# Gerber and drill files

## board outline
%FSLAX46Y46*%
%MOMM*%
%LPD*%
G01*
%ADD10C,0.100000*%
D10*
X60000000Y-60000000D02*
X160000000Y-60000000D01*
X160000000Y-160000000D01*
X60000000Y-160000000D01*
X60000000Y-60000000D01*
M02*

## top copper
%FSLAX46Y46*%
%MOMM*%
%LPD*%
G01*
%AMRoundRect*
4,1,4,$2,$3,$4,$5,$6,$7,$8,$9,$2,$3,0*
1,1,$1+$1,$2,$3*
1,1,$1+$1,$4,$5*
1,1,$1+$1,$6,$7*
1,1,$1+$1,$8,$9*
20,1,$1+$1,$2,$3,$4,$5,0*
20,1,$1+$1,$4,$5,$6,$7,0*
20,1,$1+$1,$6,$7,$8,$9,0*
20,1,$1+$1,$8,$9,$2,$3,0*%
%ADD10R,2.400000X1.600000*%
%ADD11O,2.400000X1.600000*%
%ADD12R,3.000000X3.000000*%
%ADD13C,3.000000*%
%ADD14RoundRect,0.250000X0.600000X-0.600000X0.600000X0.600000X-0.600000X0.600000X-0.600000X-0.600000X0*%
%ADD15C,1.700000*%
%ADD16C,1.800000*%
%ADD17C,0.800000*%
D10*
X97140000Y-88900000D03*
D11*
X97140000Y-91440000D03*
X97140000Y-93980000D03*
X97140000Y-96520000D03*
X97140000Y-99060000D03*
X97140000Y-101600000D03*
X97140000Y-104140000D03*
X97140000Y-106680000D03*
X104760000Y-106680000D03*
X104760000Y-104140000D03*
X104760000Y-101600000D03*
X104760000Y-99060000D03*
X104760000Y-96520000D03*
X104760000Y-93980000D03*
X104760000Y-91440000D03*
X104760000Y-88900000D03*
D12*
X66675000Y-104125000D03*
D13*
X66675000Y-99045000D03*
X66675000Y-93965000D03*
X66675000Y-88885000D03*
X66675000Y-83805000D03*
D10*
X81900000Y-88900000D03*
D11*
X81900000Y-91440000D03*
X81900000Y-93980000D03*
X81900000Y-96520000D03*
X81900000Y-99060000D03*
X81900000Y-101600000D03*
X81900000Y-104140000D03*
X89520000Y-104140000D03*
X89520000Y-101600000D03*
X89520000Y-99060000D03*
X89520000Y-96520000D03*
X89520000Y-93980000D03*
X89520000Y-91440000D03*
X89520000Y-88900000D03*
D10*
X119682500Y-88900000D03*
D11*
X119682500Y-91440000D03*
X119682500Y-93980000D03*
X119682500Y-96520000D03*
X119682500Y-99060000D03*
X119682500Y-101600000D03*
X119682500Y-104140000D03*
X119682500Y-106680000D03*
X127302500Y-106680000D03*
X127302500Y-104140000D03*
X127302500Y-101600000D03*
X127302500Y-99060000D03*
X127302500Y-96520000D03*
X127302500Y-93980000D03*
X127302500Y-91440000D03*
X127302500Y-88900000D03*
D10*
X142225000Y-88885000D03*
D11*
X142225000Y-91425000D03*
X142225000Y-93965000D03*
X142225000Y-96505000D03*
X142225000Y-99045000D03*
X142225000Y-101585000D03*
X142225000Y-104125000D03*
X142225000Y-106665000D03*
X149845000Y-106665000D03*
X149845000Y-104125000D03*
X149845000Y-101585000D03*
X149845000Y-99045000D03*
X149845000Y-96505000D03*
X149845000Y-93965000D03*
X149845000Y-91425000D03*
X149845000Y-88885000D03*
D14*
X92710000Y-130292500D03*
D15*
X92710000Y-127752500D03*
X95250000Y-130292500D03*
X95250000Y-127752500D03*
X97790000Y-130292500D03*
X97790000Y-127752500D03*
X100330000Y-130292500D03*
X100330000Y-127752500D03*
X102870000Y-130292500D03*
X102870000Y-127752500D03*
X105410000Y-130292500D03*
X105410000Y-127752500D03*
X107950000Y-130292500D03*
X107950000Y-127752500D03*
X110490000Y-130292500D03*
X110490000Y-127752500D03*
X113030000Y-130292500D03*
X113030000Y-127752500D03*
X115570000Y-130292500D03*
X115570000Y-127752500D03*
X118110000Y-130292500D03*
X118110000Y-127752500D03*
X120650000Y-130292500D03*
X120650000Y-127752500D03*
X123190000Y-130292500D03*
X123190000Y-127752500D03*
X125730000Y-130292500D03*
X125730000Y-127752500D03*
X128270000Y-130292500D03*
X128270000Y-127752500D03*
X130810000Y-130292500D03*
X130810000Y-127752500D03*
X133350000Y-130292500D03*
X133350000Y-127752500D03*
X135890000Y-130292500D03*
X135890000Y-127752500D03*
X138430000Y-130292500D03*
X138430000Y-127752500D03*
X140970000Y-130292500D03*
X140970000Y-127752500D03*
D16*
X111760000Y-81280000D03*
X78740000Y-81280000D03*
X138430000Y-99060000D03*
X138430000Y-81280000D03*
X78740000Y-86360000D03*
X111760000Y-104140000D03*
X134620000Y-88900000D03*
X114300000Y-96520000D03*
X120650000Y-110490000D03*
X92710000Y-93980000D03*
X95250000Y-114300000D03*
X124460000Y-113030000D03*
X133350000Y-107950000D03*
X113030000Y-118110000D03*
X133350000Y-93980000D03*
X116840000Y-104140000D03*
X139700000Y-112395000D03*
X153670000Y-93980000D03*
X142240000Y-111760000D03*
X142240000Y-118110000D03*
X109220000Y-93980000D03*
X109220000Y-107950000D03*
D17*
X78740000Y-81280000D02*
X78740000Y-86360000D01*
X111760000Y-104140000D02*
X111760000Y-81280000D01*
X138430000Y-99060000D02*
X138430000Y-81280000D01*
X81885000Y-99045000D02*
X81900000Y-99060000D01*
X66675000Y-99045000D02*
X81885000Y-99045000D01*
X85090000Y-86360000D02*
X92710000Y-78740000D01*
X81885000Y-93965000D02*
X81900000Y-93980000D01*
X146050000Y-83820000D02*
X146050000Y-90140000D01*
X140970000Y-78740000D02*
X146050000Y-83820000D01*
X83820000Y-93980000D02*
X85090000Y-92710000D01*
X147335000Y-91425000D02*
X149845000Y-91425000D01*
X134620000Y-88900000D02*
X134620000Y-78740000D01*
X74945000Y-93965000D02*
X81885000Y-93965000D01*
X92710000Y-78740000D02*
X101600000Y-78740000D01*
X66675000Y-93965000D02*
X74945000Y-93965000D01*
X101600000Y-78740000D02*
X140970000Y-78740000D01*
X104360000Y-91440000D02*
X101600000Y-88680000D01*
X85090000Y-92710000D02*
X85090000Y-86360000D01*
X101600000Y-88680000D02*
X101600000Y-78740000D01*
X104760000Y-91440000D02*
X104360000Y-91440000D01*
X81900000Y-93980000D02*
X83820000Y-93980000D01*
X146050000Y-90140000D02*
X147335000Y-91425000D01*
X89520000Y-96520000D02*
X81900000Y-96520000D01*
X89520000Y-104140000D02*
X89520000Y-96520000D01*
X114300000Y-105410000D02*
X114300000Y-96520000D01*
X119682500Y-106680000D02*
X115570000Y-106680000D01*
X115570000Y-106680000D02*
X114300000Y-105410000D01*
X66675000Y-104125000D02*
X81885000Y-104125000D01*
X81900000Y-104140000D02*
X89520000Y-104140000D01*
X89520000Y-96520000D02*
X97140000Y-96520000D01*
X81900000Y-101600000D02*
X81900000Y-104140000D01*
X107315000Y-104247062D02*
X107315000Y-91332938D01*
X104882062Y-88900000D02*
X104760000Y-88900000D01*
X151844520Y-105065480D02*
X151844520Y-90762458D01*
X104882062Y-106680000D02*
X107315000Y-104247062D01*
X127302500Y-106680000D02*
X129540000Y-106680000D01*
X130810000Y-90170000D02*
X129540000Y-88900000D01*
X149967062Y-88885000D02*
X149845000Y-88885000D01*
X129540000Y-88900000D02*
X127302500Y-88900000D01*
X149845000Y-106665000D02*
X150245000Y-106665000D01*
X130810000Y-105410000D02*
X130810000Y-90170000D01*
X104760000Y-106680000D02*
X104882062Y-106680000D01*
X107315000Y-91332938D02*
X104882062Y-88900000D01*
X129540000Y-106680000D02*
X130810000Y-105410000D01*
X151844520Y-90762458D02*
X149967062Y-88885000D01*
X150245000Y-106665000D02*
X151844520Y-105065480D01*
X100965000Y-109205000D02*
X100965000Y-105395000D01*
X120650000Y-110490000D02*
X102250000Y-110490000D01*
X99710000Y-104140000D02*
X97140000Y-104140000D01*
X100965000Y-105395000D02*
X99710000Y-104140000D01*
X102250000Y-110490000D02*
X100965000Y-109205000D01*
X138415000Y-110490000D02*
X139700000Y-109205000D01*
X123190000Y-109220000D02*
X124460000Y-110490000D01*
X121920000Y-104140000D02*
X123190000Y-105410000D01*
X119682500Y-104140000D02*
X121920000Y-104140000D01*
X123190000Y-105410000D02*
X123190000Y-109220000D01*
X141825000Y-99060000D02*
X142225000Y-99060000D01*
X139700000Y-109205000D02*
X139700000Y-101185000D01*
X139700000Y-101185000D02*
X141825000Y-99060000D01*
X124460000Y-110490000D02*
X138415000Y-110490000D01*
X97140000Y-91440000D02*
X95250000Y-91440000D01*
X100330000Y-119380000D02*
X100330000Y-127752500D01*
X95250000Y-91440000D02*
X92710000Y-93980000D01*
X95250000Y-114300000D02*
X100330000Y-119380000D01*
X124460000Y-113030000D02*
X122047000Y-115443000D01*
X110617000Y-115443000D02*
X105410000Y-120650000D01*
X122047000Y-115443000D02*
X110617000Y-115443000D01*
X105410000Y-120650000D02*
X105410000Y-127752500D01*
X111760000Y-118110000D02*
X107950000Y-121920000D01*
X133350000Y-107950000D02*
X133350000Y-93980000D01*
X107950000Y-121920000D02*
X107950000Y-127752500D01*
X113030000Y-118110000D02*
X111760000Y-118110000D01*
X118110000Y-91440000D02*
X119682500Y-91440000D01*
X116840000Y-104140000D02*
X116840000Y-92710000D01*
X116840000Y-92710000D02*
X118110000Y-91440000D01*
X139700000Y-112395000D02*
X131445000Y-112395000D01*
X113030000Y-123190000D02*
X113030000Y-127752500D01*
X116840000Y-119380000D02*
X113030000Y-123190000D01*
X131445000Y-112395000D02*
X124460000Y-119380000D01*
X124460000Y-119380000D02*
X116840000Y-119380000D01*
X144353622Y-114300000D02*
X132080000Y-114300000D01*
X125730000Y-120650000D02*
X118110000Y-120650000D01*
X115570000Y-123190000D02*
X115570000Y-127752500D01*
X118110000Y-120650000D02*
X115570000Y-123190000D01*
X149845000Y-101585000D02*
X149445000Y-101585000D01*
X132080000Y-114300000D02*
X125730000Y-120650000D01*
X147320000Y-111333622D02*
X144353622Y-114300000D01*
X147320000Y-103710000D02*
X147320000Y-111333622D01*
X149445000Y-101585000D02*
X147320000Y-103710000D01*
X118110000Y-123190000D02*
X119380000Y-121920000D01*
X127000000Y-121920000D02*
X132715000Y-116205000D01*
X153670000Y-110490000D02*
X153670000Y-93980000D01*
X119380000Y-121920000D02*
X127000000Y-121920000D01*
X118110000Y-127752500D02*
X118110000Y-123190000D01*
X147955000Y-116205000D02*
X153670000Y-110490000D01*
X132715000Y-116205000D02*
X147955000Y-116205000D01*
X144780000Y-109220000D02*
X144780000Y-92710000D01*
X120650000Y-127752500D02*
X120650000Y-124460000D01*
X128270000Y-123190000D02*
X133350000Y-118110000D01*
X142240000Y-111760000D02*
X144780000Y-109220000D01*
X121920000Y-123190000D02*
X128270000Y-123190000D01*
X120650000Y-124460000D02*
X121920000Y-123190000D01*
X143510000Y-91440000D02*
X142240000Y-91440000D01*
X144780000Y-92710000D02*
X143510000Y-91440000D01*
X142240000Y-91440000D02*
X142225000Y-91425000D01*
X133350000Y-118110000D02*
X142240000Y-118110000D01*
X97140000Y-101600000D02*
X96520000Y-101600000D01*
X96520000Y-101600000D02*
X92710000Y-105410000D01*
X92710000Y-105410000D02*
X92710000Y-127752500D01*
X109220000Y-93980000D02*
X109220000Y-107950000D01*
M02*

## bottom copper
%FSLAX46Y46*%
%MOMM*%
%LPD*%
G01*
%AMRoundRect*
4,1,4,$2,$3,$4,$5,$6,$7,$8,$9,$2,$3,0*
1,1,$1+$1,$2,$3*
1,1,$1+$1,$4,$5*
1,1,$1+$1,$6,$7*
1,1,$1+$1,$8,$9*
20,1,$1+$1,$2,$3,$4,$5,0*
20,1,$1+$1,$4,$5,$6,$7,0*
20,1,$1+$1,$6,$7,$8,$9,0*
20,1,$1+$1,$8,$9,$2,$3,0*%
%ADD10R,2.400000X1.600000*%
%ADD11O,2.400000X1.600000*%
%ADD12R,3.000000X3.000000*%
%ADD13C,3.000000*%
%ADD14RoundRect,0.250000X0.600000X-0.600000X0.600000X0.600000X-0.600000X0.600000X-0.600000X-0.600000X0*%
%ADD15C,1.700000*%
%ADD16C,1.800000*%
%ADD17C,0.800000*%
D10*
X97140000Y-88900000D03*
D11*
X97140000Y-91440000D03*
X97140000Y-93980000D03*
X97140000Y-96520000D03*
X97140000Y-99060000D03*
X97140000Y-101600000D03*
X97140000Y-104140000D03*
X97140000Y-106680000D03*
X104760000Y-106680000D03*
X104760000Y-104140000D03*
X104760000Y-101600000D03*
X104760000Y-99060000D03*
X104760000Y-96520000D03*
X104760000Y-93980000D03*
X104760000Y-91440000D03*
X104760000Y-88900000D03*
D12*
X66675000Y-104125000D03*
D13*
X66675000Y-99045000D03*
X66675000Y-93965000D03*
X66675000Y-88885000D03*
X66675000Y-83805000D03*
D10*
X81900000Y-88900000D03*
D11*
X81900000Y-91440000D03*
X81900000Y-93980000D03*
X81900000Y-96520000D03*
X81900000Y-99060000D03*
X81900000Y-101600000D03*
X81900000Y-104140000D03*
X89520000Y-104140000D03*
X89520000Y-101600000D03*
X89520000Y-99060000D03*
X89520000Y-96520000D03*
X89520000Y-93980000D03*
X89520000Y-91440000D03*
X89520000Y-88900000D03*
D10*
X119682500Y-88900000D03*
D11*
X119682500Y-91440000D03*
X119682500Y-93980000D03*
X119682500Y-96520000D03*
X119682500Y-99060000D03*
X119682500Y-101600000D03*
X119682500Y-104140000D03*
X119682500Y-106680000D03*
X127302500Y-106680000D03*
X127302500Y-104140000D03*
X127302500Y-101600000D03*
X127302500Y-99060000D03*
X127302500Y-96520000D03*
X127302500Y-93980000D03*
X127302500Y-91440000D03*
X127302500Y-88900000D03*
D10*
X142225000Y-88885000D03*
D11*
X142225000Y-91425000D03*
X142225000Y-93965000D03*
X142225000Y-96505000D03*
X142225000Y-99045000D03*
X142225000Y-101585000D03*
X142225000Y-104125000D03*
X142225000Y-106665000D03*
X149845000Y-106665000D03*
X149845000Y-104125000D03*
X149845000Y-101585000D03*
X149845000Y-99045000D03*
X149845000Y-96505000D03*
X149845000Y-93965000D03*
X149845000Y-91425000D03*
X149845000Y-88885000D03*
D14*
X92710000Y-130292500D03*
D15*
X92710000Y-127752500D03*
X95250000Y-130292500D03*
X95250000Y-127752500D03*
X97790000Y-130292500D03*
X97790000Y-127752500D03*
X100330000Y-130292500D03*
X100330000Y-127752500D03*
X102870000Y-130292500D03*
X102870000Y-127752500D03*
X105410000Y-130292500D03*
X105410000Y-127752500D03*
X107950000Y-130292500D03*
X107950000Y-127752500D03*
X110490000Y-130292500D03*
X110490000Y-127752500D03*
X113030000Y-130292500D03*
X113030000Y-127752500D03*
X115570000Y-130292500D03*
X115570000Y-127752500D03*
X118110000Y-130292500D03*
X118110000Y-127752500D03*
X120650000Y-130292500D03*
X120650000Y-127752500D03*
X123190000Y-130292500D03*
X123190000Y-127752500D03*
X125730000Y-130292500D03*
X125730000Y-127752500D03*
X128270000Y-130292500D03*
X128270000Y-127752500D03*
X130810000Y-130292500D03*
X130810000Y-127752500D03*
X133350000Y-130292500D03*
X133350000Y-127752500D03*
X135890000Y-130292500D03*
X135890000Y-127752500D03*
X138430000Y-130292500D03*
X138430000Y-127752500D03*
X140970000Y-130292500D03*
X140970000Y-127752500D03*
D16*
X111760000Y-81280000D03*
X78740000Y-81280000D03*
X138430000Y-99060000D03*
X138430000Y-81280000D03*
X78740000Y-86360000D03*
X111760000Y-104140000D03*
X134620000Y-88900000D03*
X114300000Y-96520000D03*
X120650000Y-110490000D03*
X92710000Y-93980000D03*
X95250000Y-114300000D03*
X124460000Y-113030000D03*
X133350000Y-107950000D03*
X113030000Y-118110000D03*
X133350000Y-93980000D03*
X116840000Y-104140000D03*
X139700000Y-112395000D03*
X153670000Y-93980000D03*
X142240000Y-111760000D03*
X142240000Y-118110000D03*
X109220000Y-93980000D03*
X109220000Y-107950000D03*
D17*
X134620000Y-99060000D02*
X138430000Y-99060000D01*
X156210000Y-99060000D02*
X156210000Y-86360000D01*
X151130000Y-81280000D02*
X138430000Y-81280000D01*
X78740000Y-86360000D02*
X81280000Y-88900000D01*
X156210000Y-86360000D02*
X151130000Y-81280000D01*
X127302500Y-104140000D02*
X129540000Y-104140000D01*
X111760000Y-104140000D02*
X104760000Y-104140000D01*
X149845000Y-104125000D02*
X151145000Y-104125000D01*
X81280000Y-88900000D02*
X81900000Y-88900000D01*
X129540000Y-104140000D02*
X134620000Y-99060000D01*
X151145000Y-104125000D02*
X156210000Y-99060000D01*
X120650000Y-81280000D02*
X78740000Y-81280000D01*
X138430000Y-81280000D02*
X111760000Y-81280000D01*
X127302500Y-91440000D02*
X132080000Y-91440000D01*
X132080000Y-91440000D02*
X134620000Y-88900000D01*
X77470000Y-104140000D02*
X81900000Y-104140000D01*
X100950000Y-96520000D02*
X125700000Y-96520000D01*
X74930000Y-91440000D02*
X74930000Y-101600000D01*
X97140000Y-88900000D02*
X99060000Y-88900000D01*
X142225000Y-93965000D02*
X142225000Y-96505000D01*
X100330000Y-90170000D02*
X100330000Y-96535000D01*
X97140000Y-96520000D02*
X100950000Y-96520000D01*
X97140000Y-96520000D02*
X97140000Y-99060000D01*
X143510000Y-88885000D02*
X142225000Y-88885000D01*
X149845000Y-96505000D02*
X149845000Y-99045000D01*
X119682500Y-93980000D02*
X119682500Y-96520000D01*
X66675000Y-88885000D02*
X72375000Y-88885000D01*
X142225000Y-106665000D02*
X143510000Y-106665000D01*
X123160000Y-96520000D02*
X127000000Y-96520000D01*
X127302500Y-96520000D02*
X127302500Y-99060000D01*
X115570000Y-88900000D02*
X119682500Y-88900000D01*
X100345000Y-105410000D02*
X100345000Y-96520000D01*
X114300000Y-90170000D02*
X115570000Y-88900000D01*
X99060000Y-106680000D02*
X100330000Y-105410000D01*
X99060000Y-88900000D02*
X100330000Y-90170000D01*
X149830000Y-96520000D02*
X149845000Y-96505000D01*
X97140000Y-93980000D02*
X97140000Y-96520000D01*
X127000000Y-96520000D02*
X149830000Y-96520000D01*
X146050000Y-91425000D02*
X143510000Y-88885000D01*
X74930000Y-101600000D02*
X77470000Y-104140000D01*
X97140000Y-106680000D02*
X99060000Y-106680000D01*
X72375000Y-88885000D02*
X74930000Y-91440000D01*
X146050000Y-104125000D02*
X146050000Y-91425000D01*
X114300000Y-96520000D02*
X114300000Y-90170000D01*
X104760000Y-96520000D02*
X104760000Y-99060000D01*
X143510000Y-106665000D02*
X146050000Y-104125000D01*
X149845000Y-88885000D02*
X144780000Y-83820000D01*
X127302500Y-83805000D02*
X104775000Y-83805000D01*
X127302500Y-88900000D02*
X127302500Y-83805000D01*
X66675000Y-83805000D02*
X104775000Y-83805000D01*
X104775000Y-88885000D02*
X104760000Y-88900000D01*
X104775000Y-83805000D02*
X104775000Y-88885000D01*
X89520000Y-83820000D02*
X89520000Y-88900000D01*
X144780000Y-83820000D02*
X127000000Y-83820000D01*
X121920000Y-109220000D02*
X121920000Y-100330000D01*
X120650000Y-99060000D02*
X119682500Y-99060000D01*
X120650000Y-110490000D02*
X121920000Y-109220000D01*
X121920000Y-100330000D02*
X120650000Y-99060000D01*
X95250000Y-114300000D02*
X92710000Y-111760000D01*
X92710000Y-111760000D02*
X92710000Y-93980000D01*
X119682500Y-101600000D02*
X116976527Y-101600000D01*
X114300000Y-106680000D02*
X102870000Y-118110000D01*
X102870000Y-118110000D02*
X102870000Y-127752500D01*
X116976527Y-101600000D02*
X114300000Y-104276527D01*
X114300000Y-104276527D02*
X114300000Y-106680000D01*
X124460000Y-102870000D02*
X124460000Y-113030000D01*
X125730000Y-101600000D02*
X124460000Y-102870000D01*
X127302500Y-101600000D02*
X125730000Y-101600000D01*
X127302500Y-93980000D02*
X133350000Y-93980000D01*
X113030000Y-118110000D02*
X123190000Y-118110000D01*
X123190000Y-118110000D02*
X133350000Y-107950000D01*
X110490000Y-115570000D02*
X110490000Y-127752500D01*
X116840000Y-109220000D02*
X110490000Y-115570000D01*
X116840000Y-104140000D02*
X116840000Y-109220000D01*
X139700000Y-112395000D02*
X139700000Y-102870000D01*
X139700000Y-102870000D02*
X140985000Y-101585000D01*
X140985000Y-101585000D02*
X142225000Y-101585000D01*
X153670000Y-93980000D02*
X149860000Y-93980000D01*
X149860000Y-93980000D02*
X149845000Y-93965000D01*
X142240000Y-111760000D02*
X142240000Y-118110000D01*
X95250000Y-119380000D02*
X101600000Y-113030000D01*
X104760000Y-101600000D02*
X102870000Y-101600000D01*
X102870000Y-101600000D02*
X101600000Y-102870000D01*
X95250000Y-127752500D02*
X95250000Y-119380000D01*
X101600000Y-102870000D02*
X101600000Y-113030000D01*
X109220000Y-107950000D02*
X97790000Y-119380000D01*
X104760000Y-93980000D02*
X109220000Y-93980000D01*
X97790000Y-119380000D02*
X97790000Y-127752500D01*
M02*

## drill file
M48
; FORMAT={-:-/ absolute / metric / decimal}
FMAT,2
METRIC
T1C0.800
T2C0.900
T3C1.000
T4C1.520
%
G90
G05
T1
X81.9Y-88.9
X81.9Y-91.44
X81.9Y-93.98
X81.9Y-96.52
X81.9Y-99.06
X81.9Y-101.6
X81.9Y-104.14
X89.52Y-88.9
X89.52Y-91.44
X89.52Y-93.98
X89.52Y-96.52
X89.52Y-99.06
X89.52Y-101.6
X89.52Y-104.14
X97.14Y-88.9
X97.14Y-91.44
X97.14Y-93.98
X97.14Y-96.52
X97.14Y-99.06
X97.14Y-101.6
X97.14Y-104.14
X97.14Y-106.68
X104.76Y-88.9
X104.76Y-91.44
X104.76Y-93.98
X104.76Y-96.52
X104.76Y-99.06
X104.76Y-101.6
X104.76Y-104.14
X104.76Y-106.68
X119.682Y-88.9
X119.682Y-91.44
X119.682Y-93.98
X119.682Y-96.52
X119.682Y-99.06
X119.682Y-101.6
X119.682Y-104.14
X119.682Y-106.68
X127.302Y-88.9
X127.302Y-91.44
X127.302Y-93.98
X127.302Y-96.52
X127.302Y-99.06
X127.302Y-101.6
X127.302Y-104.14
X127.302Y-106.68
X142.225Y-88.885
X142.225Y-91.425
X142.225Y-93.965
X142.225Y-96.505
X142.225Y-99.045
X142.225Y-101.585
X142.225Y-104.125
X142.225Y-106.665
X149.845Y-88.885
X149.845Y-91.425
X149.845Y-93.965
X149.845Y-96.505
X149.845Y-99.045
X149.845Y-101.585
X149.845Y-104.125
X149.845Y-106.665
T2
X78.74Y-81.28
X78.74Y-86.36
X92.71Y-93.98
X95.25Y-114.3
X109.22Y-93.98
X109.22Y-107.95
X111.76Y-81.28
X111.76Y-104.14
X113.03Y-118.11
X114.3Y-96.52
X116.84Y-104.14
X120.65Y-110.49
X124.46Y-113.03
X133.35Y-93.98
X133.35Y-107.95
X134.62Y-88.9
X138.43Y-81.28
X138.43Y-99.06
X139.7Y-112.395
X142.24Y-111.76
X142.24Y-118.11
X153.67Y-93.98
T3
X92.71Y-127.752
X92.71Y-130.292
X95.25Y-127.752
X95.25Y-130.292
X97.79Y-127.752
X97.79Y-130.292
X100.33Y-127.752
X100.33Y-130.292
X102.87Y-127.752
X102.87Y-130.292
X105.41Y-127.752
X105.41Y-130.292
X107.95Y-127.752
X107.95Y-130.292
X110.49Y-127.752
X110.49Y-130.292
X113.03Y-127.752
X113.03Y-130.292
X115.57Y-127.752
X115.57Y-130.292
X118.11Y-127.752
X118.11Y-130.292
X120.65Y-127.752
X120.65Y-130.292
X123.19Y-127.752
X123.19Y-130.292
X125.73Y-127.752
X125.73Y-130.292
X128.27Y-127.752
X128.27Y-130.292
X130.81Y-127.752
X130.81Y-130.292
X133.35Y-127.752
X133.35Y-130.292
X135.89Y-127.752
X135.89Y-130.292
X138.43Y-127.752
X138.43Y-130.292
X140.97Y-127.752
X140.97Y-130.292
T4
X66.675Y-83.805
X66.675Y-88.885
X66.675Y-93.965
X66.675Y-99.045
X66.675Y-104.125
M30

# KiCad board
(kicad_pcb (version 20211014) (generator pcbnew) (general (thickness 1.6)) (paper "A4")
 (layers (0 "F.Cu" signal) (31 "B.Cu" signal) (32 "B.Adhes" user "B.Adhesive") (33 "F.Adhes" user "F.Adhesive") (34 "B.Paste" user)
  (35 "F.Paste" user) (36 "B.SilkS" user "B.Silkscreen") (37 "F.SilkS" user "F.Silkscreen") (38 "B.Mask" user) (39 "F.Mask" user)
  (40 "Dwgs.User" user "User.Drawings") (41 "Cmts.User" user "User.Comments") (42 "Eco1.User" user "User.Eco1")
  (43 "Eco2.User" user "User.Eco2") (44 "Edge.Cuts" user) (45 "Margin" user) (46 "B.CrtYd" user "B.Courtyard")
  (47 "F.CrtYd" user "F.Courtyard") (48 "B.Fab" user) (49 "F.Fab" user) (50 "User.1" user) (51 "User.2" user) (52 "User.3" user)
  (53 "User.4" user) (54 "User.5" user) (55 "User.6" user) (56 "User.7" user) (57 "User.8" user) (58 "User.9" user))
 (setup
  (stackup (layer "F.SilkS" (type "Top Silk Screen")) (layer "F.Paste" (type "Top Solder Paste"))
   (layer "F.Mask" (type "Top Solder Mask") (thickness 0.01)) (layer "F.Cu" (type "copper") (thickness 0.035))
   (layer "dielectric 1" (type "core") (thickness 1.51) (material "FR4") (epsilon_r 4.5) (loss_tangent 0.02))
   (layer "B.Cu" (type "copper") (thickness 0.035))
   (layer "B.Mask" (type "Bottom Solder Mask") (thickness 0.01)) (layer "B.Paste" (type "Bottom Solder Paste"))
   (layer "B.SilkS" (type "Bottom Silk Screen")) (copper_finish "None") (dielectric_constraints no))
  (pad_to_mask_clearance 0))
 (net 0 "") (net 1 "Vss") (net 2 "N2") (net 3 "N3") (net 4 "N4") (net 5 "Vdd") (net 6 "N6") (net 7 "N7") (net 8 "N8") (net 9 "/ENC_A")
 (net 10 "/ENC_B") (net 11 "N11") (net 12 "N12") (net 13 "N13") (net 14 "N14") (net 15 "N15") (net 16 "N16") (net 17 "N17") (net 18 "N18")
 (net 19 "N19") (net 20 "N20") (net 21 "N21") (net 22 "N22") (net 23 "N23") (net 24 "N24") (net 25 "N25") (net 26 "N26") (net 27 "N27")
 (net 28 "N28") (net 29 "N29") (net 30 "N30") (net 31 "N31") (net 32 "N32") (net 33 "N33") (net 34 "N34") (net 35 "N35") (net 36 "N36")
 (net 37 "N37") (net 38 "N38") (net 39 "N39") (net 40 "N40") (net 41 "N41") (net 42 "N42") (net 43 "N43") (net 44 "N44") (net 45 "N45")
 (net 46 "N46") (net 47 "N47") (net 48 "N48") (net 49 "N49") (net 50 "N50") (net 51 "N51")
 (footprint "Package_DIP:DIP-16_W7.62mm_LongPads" (layer "F.Cu") (at 97.14 88.9)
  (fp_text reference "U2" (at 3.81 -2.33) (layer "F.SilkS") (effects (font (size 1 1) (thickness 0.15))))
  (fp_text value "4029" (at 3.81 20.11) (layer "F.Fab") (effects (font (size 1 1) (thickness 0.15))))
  (pad "1" thru_hole rect (at 0 0) (size 2.4 1.6) (drill 0.8) (layers *.Cu *.Mask) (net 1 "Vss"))
  (pad "2" thru_hole oval (at 0 2.54) (size 2.4 1.6) (drill 0.8) (layers *.Cu *.Mask) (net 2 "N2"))
  (pad "3" thru_hole oval (at 0 5.08) (size 2.4 1.6) (drill 0.8) (layers *.Cu *.Mask) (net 1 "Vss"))
  (pad "4" thru_hole oval (at 0 7.62) (size 2.4 1.6) (drill 0.8) (layers *.Cu *.Mask) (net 1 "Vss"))
  (pad "5" thru_hole oval (at 0 10.16) (size 2.4 1.6) (drill 0.8) (layers *.Cu *.Mask) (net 1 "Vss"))
  (pad "6" thru_hole oval (at 0 12.7) (size 2.4 1.6) (drill 0.8) (layers *.Cu *.Mask) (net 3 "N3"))
  (pad "7" thru_hole oval (at 0 15.24) (size 2.4 1.6) (drill 0.8) (layers *.Cu *.Mask) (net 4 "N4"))
  (pad "8" thru_hole oval (at 0 17.78) (size 2.4 1.6) (drill 0.8) (layers *.Cu *.Mask) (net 1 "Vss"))
  (pad "9" thru_hole oval (at 7.62 17.78) (size 2.4 1.6) (drill 0.8) (layers *.Cu *.Mask) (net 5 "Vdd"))
  (pad "10" thru_hole oval (at 7.62 15.24) (size 2.4 1.6) (drill 0.8) (layers *.Cu *.Mask) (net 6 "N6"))
  (pad "11" thru_hole oval (at 7.62 12.7) (size 2.4 1.6) (drill 0.8) (layers *.Cu *.Mask) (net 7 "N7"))
  (pad "12" thru_hole oval (at 7.62 10.16) (size 2.4 1.6) (drill 0.8) (layers *.Cu *.Mask) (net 1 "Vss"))
  (pad "13" thru_hole oval (at 7.62 7.62) (size 2.4 1.6) (drill 0.8) (layers *.Cu *.Mask) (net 1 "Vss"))
  (pad "14" thru_hole oval (at 7.62 5.08) (size 2.4 1.6) (drill 0.8) (layers *.Cu *.Mask) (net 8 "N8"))
  (pad "15" thru_hole oval (at 7.62 2.54) (size 2.4 1.6) (drill 0.8) (layers *.Cu *.Mask) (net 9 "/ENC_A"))
  (pad "16" thru_hole oval (at 7.62 0) (size 2.4 1.6) (drill 0.8) (layers *.Cu *.Mask) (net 5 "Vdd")))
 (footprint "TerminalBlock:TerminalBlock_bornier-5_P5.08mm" (layer "F.Cu") (at 66.675 104.125 90)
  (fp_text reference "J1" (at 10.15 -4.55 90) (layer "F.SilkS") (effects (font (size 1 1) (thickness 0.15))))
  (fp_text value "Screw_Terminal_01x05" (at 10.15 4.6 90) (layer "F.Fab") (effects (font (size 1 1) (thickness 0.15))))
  (pad "1" thru_hole rect (at 0 0 90) (size 3 3) (drill 1.52) (layers *.Cu *.Mask) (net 1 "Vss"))
  (pad "2" thru_hole circle (at 5.08 0 90) (size 3 3) (drill 1.52) (layers *.Cu *.Mask) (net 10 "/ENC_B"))
  (pad "3" thru_hole circle (at 10.16 0 90) (size 3 3) (drill 1.52) (layers *.Cu *.Mask) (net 9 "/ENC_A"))
  (pad "4" thru_hole circle (at 15.24 0 90) (size 3 3) (drill 1.52) (layers *.Cu *.Mask) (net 1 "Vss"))
  (pad "5" thru_hole circle (at 20.32 0 90) (size 3 3) (drill 1.52) (layers *.Cu *.Mask) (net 5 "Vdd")))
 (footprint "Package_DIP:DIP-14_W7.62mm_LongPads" (layer "F.Cu") (at 81.9 88.9)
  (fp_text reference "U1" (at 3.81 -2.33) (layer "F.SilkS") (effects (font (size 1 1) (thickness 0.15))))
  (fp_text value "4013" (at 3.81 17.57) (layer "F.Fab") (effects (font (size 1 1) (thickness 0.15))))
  (pad "1" thru_hole rect (at 0 0) (size 2.4 1.6) (drill 0.8) (layers *.Cu *.Mask) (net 6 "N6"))
  (pad "2" thru_hole oval (at 0 2.54) (size 2.4 1.6) (drill 0.8) (layers *.Cu *.Mask) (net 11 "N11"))
  (pad "3" thru_hole oval (at 0 5.08) (size 2.4 1.6) (drill 0.8) (layers *.Cu *.Mask) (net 9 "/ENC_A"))
  (pad "4" thru_hole oval (at 0 7.62) (size 2.4 1.6) (drill 0.8) (layers *.Cu *.Mask) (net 1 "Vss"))
  (pad "5" thru_hole oval (at 0 10.16) (size 2.4 1.6) (drill 0.8) (layers *.Cu *.Mask) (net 10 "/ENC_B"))
  (pad "6" thru_hole oval (at 0 12.7) (size 2.4 1.6) (drill 0.8) (layers *.Cu *.Mask) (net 1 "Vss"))
  (pad "7" thru_hole oval (at 0 15.24) (size 2.4 1.6) (drill 0.8) (layers *.Cu *.Mask) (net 1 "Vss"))
  (pad "8" thru_hole oval (at 7.62 15.24) (size 2.4 1.6) (drill 0.8) (layers *.Cu *.Mask) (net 1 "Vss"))
  (pad "9" thru_hole oval (at 7.62 12.7) (size 2.4 1.6) (drill 0.8) (layers *.Cu *.Mask) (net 1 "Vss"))
  (pad "10" thru_hole oval (at 7.62 10.16) (size 2.4 1.6) (drill 0.8) (layers *.Cu *.Mask) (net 1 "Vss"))
  (pad "11" thru_hole oval (at 7.62 7.62) (size 2.4 1.6) (drill 0.8) (layers *.Cu *.Mask) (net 1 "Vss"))
  (pad "12" thru_hole oval (at 7.62 5.08) (size 2.4 1.6) (drill 0.8) (layers *.Cu *.Mask) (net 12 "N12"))
  (pad "13" thru_hole oval (at 7.62 2.54) (size 2.4 1.6) (drill 0.8) (layers *.Cu *.Mask) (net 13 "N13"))
  (pad "14" thru_hole oval (at 7.62 0) (size 2.4 1.6) (drill 0.8) (layers *.Cu *.Mask) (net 5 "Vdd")))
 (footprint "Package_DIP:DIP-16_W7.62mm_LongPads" (layer "F.Cu") (at 119.6825 88.9)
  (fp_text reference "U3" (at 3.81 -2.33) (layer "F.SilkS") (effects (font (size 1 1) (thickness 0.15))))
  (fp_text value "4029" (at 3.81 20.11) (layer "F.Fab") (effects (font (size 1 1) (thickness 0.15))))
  (pad "1" thru_hole rect (at 0 0) (size 2.4 1.6) (drill 0.8) (layers *.Cu *.Mask) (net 1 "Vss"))
  (pad "2" thru_hole oval (at 0 2.54) (size 2.4 1.6) (drill 0.8) (layers *.Cu *.Mask) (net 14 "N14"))
  (pad "3" thru_hole oval (at 0 5.08) (size 2.4 1.6) (drill 0.8) (layers *.Cu *.Mask) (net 1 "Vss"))
  (pad "4" thru_hole oval (at 0 7.62) (size 2.4 1.6) (drill 0.8) (layers *.Cu *.Mask) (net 1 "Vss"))
  (pad "5" thru_hole oval (at 0 10.16) (size 2.4 1.6) (drill 0.8) (layers *.Cu *.Mask) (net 4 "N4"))
  (pad "6" thru_hole oval (at 0 12.7) (size 2.4 1.6) (drill 0.8) (layers *.Cu *.Mask) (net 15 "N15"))
  (pad "7" thru_hole oval (at 0 15.24) (size 2.4 1.6) (drill 0.8) (layers *.Cu *.Mask) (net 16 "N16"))
  (pad "8" thru_hole oval (at 0 17.78) (size 2.4 1.6) (drill 0.8) (layers *.Cu *.Mask) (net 1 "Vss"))
  (pad "9" thru_hole oval (at 7.62 17.78) (size 2.4 1.6) (drill 0.8) (layers *.Cu *.Mask) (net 5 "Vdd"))
  (pad "10" thru_hole oval (at 7.62 15.24) (size 2.4 1.6) (drill 0.8) (layers *.Cu *.Mask) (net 6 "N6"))
  (pad "11" thru_hole oval (at 7.62 12.7) (size 2.4 1.6) (drill 0.8) (layers *.Cu *.Mask) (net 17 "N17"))
  (pad "12" thru_hole oval (at 7.62 10.16) (size 2.4 1.6) (drill 0.8) (layers *.Cu *.Mask) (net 1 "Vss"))
  (pad "13" thru_hole oval (at 7.62 7.62) (size 2.4 1.6) (drill 0.8) (layers *.Cu *.Mask) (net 1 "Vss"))
  (pad "14" thru_hole oval (at 7.62 5.08) (size 2.4 1.6) (drill 0.8) (layers *.Cu *.Mask) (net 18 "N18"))
  (pad "15" thru_hole oval (at 7.62 2.54) (size 2.4 1.6) (drill 0.8) (layers *.Cu *.Mask) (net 9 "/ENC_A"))
  (pad "16" thru_hole oval (at 7.62 0) (size 2.4 1.6) (drill 0.8) (layers *.Cu *.Mask) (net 5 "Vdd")))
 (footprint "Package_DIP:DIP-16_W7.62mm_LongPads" (layer "F.Cu") (at 142.225 88.885)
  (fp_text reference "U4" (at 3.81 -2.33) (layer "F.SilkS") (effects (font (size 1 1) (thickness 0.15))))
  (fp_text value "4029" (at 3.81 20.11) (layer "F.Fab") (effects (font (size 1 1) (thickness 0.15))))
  (pad "1" thru_hole rect (at 0 0) (size 2.4 1.6) (drill 0.8) (layers *.Cu *.Mask) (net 1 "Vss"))
  (pad "2" thru_hole oval (at 0 2.54) (size 2.4 1.6) (drill 0.8) (layers *.Cu *.Mask) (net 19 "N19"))
  (pad "3" thru_hole oval (at 0 5.08) (size 2.4 1.6) (drill 0.8) (layers *.Cu *.Mask) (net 1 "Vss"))
  (pad "4" thru_hole oval (at 0 7.62) (size 2.4 1.6) (drill 0.8) (layers *.Cu *.Mask) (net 1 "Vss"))
  (pad "5" thru_hole oval (at 0 10.16) (size 2.4 1.6) (drill 0.8) (layers *.Cu *.Mask) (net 16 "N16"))
  (pad "6" thru_hole oval (at 0 12.7) (size 2.4 1.6) (drill 0.8) (layers *.Cu *.Mask) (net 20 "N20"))
  (pad "7" thru_hole oval (at 0 15.24) (size 2.4 1.6) (drill 0.8) (layers *.Cu *.Mask) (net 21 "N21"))
  (pad "8" thru_hole oval (at 0 17.78) (size 2.4 1.6) (drill 0.8) (layers *.Cu *.Mask) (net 1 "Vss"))
  (pad "9" thru_hole oval (at 7.62 17.78) (size 2.4 1.6) (drill 0.8) (layers *.Cu *.Mask) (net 5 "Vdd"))
  (pad "10" thru_hole oval (at 7.62 15.24) (size 2.4 1.6) (drill 0.8) (layers *.Cu *.Mask) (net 6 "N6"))
  (pad "11" thru_hole oval (at 7.62 12.7) (size 2.4 1.6) (drill 0.8) (layers *.Cu *.Mask) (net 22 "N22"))
  (pad "12" thru_hole oval (at 7.62 10.16) (size 2.4 1.6) (drill 0.8) (layers *.Cu *.Mask) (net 1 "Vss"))
  (pad "13" thru_hole oval (at 7.62 7.62) (size 2.4 1.6) (drill 0.8) (layers *.Cu *.Mask) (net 1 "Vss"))
  (pad "14" thru_hole oval (at 7.62 5.08) (size 2.4 1.6) (drill 0.8) (layers *.Cu *.Mask) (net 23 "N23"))
  (pad "15" thru_hole oval (at 7.62 2.54) (size 2.4 1.6) (drill 0.8) (layers *.Cu *.Mask) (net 9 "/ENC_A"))
  (pad "16" thru_hole oval (at 7.62 0) (size 2.4 1.6) (drill 0.8) (layers *.Cu *.Mask) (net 5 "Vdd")))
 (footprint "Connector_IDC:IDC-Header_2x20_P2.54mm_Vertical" (layer "F.Cu") (at 92.71 130.2925 90)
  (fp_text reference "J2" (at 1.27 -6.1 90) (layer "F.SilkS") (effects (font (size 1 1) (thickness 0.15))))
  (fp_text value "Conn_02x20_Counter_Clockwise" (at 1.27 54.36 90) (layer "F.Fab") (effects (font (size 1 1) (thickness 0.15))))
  (pad "1" thru_hole roundrect (at 0 0 90) (size 1.7 1.7) (drill 1) (layers *.Cu *.Mask) (roundrect_rratio 0.147059) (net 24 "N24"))
  (pad "2" thru_hole circle (at 2.54 0 90) (size 1.7 1.7) (drill 1) (layers *.Cu *.Mask) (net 3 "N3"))
  (pad "3" thru_hole circle (at 0 2.54 90) (size 1.7 1.7) (drill 1) (layers *.Cu *.Mask) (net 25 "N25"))
  (pad "4" thru_hole circle (at 2.54 2.54 90) (size 1.7 1.7) (drill 1) (layers *.Cu *.Mask) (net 7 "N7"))
  (pad "5" thru_hole circle (at 0 5.08 90) (size 1.7 1.7) (drill 1) (layers *.Cu *.Mask) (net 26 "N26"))
  (pad "6" thru_hole circle (at 2.54 5.08 90) (size 1.7 1.7) (drill 1) (layers *.Cu *.Mask) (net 8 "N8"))
  (pad "7" thru_hole circle (at 0 7.62 90) (size 1.7 1.7) (drill 1) (layers *.Cu *.Mask) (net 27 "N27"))
  (pad "8" thru_hole circle (at 2.54 7.62 90) (size 1.7 1.7) (drill 1) (layers *.Cu *.Mask) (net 2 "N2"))
  (pad "9" thru_hole circle (at 0 10.16 90) (size 1.7 1.7) (drill 1) (layers *.Cu *.Mask) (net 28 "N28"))
  (pad "10" thru_hole circle (at 2.54 10.16 90) (size 1.7 1.7) (drill 1) (layers *.Cu *.Mask) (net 15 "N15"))
  (pad "11" thru_hole circle (at 0 12.7 90) (size 1.7 1.7) (drill 1) (layers *.Cu *.Mask) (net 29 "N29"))
  (pad "12" thru_hole circle (at 2.54 12.7 90) (size 1.7 1.7) (drill 1) (layers *.Cu *.Mask) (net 17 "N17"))
  (pad "13" thru_hole circle (at 0 15.24 90) (size 1.7 1.7) (drill 1) (layers *.Cu *.Mask) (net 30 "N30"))
  (pad "14" thru_hole circle (at 2.54 15.24 90) (size 1.7 1.7) (drill 1) (layers *.Cu *.Mask) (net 18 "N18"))
  (pad "15" thru_hole circle (at 0 17.78 90) (size 1.7 1.7) (drill 1) (layers *.Cu *.Mask) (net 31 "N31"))
  (pad "16" thru_hole circle (at 2.54 17.78 90) (size 1.7 1.7) (drill 1) (layers *.Cu *.Mask) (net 14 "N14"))
  (pad "17" thru_hole circle (at 0 20.32 90) (size 1.7 1.7) (drill 1) (layers *.Cu *.Mask) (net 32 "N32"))
  (pad "18" thru_hole circle (at 2.54 20.32 90) (size 1.7 1.7) (drill 1) (layers *.Cu *.Mask) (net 20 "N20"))
  (pad "19" thru_hole circle (at 0 22.86 90) (size 1.7 1.7) (drill 1) (layers *.Cu *.Mask) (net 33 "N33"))
  (pad "20" thru_hole circle (at 2.54 22.86 90) (size 1.7 1.7) (drill 1) (layers *.Cu *.Mask) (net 22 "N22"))
  (pad "21" thru_hole circle (at 0 25.4 90) (size 1.7 1.7) (drill 1) (layers *.Cu *.Mask) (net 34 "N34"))
  (pad "22" thru_hole circle (at 2.54 25.4 90) (size 1.7 1.7) (drill 1) (layers *.Cu *.Mask) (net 23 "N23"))
  (pad "23" thru_hole circle (at 0 27.94 90) (size 1.7 1.7) (drill 1) (layers *.Cu *.Mask) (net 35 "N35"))
  (pad "24" thru_hole circle (at 2.54 27.94 90) (size 1.7 1.7) (drill 1) (layers *.Cu *.Mask) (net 19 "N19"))
  (pad "25" thru_hole circle (at 0 30.48 90) (size 1.7 1.7) (drill 1) (layers *.Cu *.Mask) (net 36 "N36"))
  (pad "26" thru_hole circle (at 2.54 30.48 90) (size 1.7 1.7) (drill 1) (layers *.Cu *.Mask) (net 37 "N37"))
  (pad "27" thru_hole circle (at 0 33.02 90) (size 1.7 1.7) (drill 1) (layers *.Cu *.Mask) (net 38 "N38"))
  (pad "28" thru_hole circle (at 2.54 33.02 90) (size 1.7 1.7) (drill 1) (layers *.Cu *.Mask) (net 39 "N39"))
  (pad "29" thru_hole circle (at 0 35.56 90) (size 1.7 1.7) (drill 1) (layers *.Cu *.Mask) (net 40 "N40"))
  (pad "30" thru_hole circle (at 2.54 35.56 90) (size 1.7 1.7) (drill 1) (layers *.Cu *.Mask) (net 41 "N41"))
  (pad "31" thru_hole circle (at 0 38.1 90) (size 1.7 1.7) (drill 1) (layers *.Cu *.Mask) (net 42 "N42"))
  (pad "32" thru_hole circle (at 2.54 38.1 90) (size 1.7 1.7) (drill 1) (layers *.Cu *.Mask) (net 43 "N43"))
  (pad "33" thru_hole circle (at 0 40.64 90) (size 1.7 1.7) (drill 1) (layers *.Cu *.Mask) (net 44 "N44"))
  (pad "34" thru_hole circle (at 2.54 40.64 90) (size 1.7 1.7) (drill 1) (layers *.Cu *.Mask) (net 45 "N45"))
  (pad "35" thru_hole circle (at 0 43.18 90) (size 1.7 1.7) (drill 1) (layers *.Cu *.Mask) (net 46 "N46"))
  (pad "36" thru_hole circle (at 2.54 43.18 90) (size 1.7 1.7) (drill 1) (layers *.Cu *.Mask) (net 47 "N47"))
  (pad "37" thru_hole circle (at 0 45.72 90) (size 1.7 1.7) (drill 1) (layers *.Cu *.Mask) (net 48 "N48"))
  (pad "38" thru_hole circle (at 2.54 45.72 90) (size 1.7 1.7) (drill 1) (layers *.Cu *.Mask) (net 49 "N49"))
  (pad "39" thru_hole circle (at 0 48.26 90) (size 1.7 1.7) (drill 1) (layers *.Cu *.Mask) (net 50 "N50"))
  (pad "40" thru_hole circle (at 2.54 48.26 90) (size 1.7 1.7) (drill 1) (layers *.Cu *.Mask) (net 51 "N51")))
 (gr_rect (start 60 60) (end 160 160) (layer "Edge.Cuts") (width 0.1) (fill none))
 (segment (start 78.74 81.28) (end 78.74 86.36) (width 0.8) (layer "F.Cu") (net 6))
 (segment (start 111.76 104.14) (end 111.76 81.28) (width 0.8) (layer "F.Cu") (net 6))
 (segment (start 138.43 99.06) (end 138.43 81.28) (width 0.8) (layer "F.Cu") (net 6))
 (via (at 111.76 81.28) (size 1.8) (drill 0.9) (layers "F.Cu" "B.Cu") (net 6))
 (via (at 78.74 81.28) (size 1.8) (drill 0.9) (layers "F.Cu" "B.Cu") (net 6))
 (via (at 138.43 99.06) (size 1.8) (drill 0.9) (layers "F.Cu" "B.Cu") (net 6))
 (via (at 138.43 81.28) (size 1.8) (drill 0.9) (layers "F.Cu" "B.Cu") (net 6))
 (via (at 78.74 86.36) (size 1.8) (drill 0.9) (layers "F.Cu" "B.Cu") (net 6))
 (via (at 111.76 104.14) (size 1.8) (drill 0.9) (layers "F.Cu" "B.Cu") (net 6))
 (segment (start 134.62 99.06) (end 138.43 99.06) (width 0.8) (layer "B.Cu") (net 6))
 (segment (start 156.21 99.06) (end 156.21 86.36) (width 0.8) (layer "B.Cu") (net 6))
 (segment (start 151.13 81.28) (end 138.43 81.28) (width 0.8) (layer "B.Cu") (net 6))
 (segment (start 78.74 86.36) (end 81.28 88.9) (width 0.8) (layer "B.Cu") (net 6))
 (segment (start 156.21 86.36) (end 151.13 81.28) (width 0.8) (layer "B.Cu") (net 6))
 (segment (start 127.3025 104.14) (end 129.54 104.14) (width 0.8) (layer "B.Cu") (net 6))
 (segment (start 111.76 104.14) (end 104.76 104.14) (width 0.8) (layer "B.Cu") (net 6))
 (segment (start 149.845 104.125) (end 151.145 104.125) (width 0.8) (layer "B.Cu") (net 6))
 (segment (start 81.28 88.9) (end 81.9 88.9) (width 0.8) (layer "B.Cu") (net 6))
 (segment (start 129.54 104.14) (end 134.62 99.06) (width 0.8) (layer "B.Cu") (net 6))
 (segment (start 151.145 104.125) (end 156.21 99.06) (width 0.8) (layer "B.Cu") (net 6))
 (segment (start 120.65 81.28) (end 78.74 81.28) (width 0.8) (layer "B.Cu") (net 6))
 (segment (start 138.43 81.28) (end 111.76 81.28) (width 0.8) (layer "B.Cu") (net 6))
 (segment (start 81.885 99.045) (end 81.9 99.06) (width 0.8) (layer "F.Cu") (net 10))
 (segment (start 66.675 99.045) (end 81.885 99.045) (width 0.8) (layer "F.Cu") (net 10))
 (segment (start 85.09 86.36) (end 92.71 78.74) (width 0.8) (layer "F.Cu") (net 9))
 (segment (start 81.885 93.965) (end 81.9 93.98) (width 0.8) (layer "F.Cu") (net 9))
 (segment (start 146.05 83.82) (end 146.05 90.14) (width 0.8) (layer "F.Cu") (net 9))
 (segment (start 140.97 78.74) (end 146.05 83.82) (width 0.8) (layer "F.Cu") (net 9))
 (segment (start 83.82 93.98) (end 85.09 92.71) (width 0.8) (layer "F.Cu") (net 9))
 (segment (start 147.335 91.425) (end 149.845 91.425) (width 0.8) (layer "F.Cu") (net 9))
 (segment (start 134.62 88.9) (end 134.62 78.74) (width 0.8) (layer "F.Cu") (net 9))
 (segment (start 74.945 93.965) (end 81.885 93.965) (width 0.8) (layer "F.Cu") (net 9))
 (segment (start 92.71 78.74) (end 101.6 78.74) (width 0.8) (layer "F.Cu") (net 9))
 (segment (start 66.675 93.965) (end 74.945 93.965) (width 0.8) (layer "F.Cu") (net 9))
 (segment (start 101.6 78.74) (end 140.97 78.74) (width 0.8) (layer "F.Cu") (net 9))
 (segment (start 104.36 91.44) (end 101.6 88.68) (width 0.8) (layer "F.Cu") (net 9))
 (segment (start 85.09 92.71) (end 85.09 86.36) (width 0.8) (layer "F.Cu") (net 9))
 (segment (start 101.6 88.68) (end 101.6 78.74) (width 0.8) (layer "F.Cu") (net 9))
 (segment (start 104.76 91.44) (end 104.36 91.44) (width 0.8) (layer "F.Cu") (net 9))
 (segment (start 81.9 93.98) (end 83.82 93.98) (width 0.8) (layer "F.Cu") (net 9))
 (segment (start 146.05 90.14) (end 147.335 91.425) (width 0.8) (layer "F.Cu") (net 9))
 (via (at 134.62 88.9) (size 1.8) (drill 0.9) (layers "F.Cu" "B.Cu") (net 9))
 (segment (start 127.3025 91.44) (end 132.08 91.44) (width 0.8) (layer "B.Cu") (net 9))
 (segment (start 132.08 91.44) (end 134.62 88.9) (width 0.8) (layer "B.Cu") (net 9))
 (segment (start 89.52 96.52) (end 81.9 96.52) (width 0.8) (layer "F.Cu") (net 1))
 (segment (start 89.52 104.14) (end 89.52 96.52) (width 0.8) (layer "F.Cu") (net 1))
 (segment (start 114.3 105.41) (end 114.3 96.52) (width 0.8) (layer "F.Cu") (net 1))
 (segment (start 119.6825 106.68) (end 115.57 106.68) (width 0.8) (layer "F.Cu") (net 1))
 (segment (start 115.57 106.68) (end 114.3 105.41) (width 0.8) (layer "F.Cu") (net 1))
 (segment (start 66.675 104.125) (end 81.885 104.125) (width 0.8) (layer "F.Cu") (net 1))
 (segment (start 81.9 104.14) (end 89.52 104.14) (width 0.8) (layer "F.Cu") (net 1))
 (segment (start 89.52 96.52) (end 97.14 96.52) (width 0.8) (layer "F.Cu") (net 1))
 (segment (start 81.9 101.6) (end 81.9 104.14) (width 0.8) (layer "F.Cu") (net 1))
 (via (at 114.3 96.52) (size 1.8) (drill 0.9) (layers "F.Cu" "B.Cu") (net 1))
 (segment (start 77.47 104.14) (end 81.9 104.14) (width 0.8) (layer "B.Cu") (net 1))
 (segment (start 100.95 96.52) (end 125.7 96.52) (width 0.8) (layer "B.Cu") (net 1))
 (segment (start 74.93 91.44) (end 74.93 101.6) (width 0.8) (layer "B.Cu") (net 1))
 (segment (start 97.14 88.9) (end 99.06 88.9) (width 0.8) (layer "B.Cu") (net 1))
 (segment (start 142.225 93.965) (end 142.225 96.505) (width 0.8) (layer "B.Cu") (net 1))
 (segment (start 100.33 90.17) (end 100.33 96.535) (width 0.8) (layer "B.Cu") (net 1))
 (segment (start 97.14 96.52) (end 100.95 96.52) (width 0.8) (layer "B.Cu") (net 1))
 (segment (start 97.14 96.52) (end 97.14 99.06) (width 0.8) (layer "B.Cu") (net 1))
 (segment (start 143.51 88.885) (end 142.225 88.885) (width 0.8) (layer "B.Cu") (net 1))
 (segment (start 149.845 96.505) (end 149.845 99.045) (width 0.8) (layer "B.Cu") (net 1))
 (segment (start 119.6825 93.98) (end 119.6825 96.52) (width 0.8) (layer "B.Cu") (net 1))
 (segment (start 66.675 88.885) (end 72.375 88.885) (width 0.8) (layer "B.Cu") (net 1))
 (segment (start 142.225 106.665) (end 143.51 106.665) (width 0.8) (layer "B.Cu") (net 1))
 (segment (start 123.16 96.52) (end 127 96.52) (width 0.8) (layer "B.Cu") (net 1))
 (segment (start 127.3025 96.52) (end 127.3025 99.06) (width 0.8) (layer "B.Cu") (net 1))
 (segment (start 115.57 88.9) (end 119.6825 88.9) (width 0.8) (layer "B.Cu") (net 1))
 (segment (start 100.345 105.41) (end 100.345 96.52) (width 0.8) (layer "B.Cu") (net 1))
 (segment (start 114.3 90.17) (end 115.57 88.9) (width 0.8) (layer "B.Cu") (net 1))
 (segment (start 99.06 106.68) (end 100.33 105.41) (width 0.8) (layer "B.Cu") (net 1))
 (segment (start 99.06 88.9) (end 100.33 90.17) (width 0.8) (layer "B.Cu") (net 1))
 (segment (start 149.83 96.52) (end 149.845 96.505) (width 0.8) (layer "B.Cu") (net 1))
 (segment (start 97.14 93.98) (end 97.14 96.52) (width 0.8) (layer "B.Cu") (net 1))
 (segment (start 127 96.52) (end 149.83 96.52) (width 0.8) (layer "B.Cu") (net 1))
 (segment (start 146.05 91.425) (end 143.51 88.885) (width 0.8) (layer "B.Cu") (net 1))
 (segment (start 74.93 101.6) (end 77.47 104.14) (width 0.8) (layer "B.Cu") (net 1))
 (segment (start 97.14 106.68) (end 99.06 106.68) (width 0.8) (layer "B.Cu") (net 1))
 (segment (start 72.375 88.885) (end 74.93 91.44) (width 0.8) (layer "B.Cu") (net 1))
 (segment (start 146.05 104.125) (end 146.05 91.425) (width 0.8) (layer "B.Cu") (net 1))
 (segment (start 114.3 96.52) (end 114.3 90.17) (width 0.8) (layer "B.Cu") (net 1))
 (segment (start 104.76 96.52) (end 104.76 99.06) (width 0.8) (layer "B.Cu") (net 1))
 (segment (start 143.51 106.665) (end 146.05 104.125) (width 0.8) (layer "B.Cu") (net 1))
 (segment (start 107.315 104.247062) (end 107.315 91.332938) (width 0.8) (layer "F.Cu") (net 5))
 (segment (start 104.882062 88.9) (end 104.76 88.9) (width 0.8) (layer "F.Cu") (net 5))
 (segment (start 151.84452 105.06548) (end 151.84452 90.762458) (width 0.8) (layer "F.Cu") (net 5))
 (segment (start 104.882062 106.68) (end 107.315 104.247062) (width 0.8) (layer "F.Cu") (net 5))
 (segment (start 127.3025 106.68) (end 129.54 106.68) (width 0.8) (layer "F.Cu") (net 5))
 (segment (start 130.81 90.17) (end 129.54 88.9) (width 0.8) (layer "F.Cu") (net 5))
 (segment (start 149.967062 88.885) (end 149.845 88.885) (width 0.8) (layer "F.Cu") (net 5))
 (segment (start 129.54 88.9) (end 127.3025 88.9) (width 0.8) (layer "F.Cu") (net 5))
 (segment (start 149.845 106.665) (end 150.245 106.665) (width 0.8) (layer "F.Cu") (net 5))
 (segment (start 130.81 105.41) (end 130.81 90.17) (width 0.8) (layer "F.Cu") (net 5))
 (segment (start 104.76 106.68) (end 104.882062 106.68) (width 0.8) (layer "F.Cu") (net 5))
 (segment (start 107.315 91.332938) (end 104.882062 88.9) (width 0.8) (layer "F.Cu") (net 5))
 (segment (start 129.54 106.68) (end 130.81 105.41) (width 0.8) (layer "F.Cu") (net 5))
 (segment (start 151.84452 90.762458) (end 149.967062 88.885) (width 0.8) (layer "F.Cu") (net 5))
 (segment (start 150.245 106.665) (end 151.84452 105.06548) (width 0.8) (layer "F.Cu") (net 5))
 (segment (start 149.845 88.885) (end 144.78 83.82) (width 0.8) (layer "B.Cu") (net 5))
 (segment (start 127.3025 83.805) (end 104.775 83.805) (width 0.8) (layer "B.Cu") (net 5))
 (segment (start 127.3025 88.9) (end 127.3025 83.805) (width 0.8) (layer "B.Cu") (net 5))
 (segment (start 66.675 83.805) (end 104.775 83.805) (width 0.8) (layer "B.Cu") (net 5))
 (segment (start 104.775 88.885) (end 104.76 88.9) (width 0.8) (layer "B.Cu") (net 5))
 (segment (start 104.775 83.805) (end 104.775 88.885) (width 0.8) (layer "B.Cu") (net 5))
 (segment (start 89.52 83.82) (end 89.52 88.9) (width 0.8) (layer "B.Cu") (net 5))
 (segment (start 144.78 83.82) (end 127 83.82) (width 0.8) (layer "B.Cu") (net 5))
 (segment (start 100.965 109.205) (end 100.965 105.395) (width 0.8) (layer "F.Cu") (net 4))
 (segment (start 120.65 110.49) (end 102.25 110.49) (width 0.8) (layer "F.Cu") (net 4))
 (segment (start 99.71 104.14) (end 97.14 104.14) (width 0.8) (layer "F.Cu") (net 4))
 (segment (start 100.965 105.395) (end 99.71 104.14) (width 0.8) (layer "F.Cu") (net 4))
 (segment (start 102.25 110.49) (end 100.965 109.205) (width 0.8) (layer "F.Cu") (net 4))
 (via (at 120.65 110.49) (size 1.8) (drill 0.9) (layers "F.Cu" "B.Cu") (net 4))
 (segment (start 121.92 109.22) (end 121.92 100.33) (width 0.8) (layer "B.Cu") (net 4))
 (segment (start 120.65 99.06) (end 119.6825 99.06) (width 0.8) (layer "B.Cu") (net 4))
 (segment (start 120.65 110.49) (end 121.92 109.22) (width 0.8) (layer "B.Cu") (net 4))
 (segment (start 121.92 100.33) (end 120.65 99.06) (width 0.8) (layer "B.Cu") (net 4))
 (segment (start 138.415 110.49) (end 139.7 109.205) (width 0.8) (layer "F.Cu") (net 16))
 (segment (start 123.19 109.22) (end 124.46 110.49) (width 0.8) (layer "F.Cu") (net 16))
 (segment (start 121.92 104.14) (end 123.19 105.41) (width 0.8) (layer "F.Cu") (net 16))
 (segment (start 119.6825 104.14) (end 121.92 104.14) (width 0.8) (layer "F.Cu") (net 16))
 (segment (start 123.19 105.41) (end 123.19 109.22) (width 0.8) (layer "F.Cu") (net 16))
 (segment (start 141.825 99.06) (end 142.225 99.06) (width 0.8) (layer "F.Cu") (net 16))
 (segment (start 139.7 109.205) (end 139.7 101.185) (width 0.8) (layer "F.Cu") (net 16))
 (segment (start 139.7 101.185) (end 141.825 99.06) (width 0.8) (layer "F.Cu") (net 16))
 (segment (start 124.46 110.49) (end 138.415 110.49) (width 0.8) (layer "F.Cu") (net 16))
 (segment (start 97.14 91.44) (end 95.25 91.44) (width 0.8) (layer "F.Cu") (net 2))
 (segment (start 100.33 119.38) (end 100.33 127.7525) (width 0.8) (layer "F.Cu") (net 2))
 (segment (start 95.25 91.44) (end 92.71 93.98) (width 0.8) (layer "F.Cu") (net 2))
 (segment (start 95.25 114.3) (end 100.33 119.38) (width 0.8) (layer "F.Cu") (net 2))
 (via (at 92.71 93.98) (size 1.8) (drill 0.9) (layers "F.Cu" "B.Cu") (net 2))
 (via (at 95.25 114.3) (size 1.8) (drill 0.9) (layers "F.Cu" "B.Cu") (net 2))
 (segment (start 95.25 114.3) (end 92.71 111.76) (width 0.8) (layer "B.Cu") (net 2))
 (segment (start 92.71 111.76) (end 92.71 93.98) (width 0.8) (layer "B.Cu") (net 2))
 (segment (start 119.6825 101.6) (end 116.976527 101.6) (width 0.8) (layer "B.Cu") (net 15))
 (segment (start 114.3 106.68) (end 102.87 118.11) (width 0.8) (layer "B.Cu") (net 15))
 (segment (start 102.87 118.11) (end 102.87 127.7525) (width 0.8) (layer "B.Cu") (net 15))
 (segment (start 116.976527 101.6) (end 114.3 104.276527) (width 0.8) (layer "B.Cu") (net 15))
 (segment (start 114.3 104.276527) (end 114.3 106.68) (width 0.8) (layer "B.Cu") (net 15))
 (segment (start 124.46 113.03) (end 122.047 115.443) (width 0.8) (layer "F.Cu") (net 17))
 (segment (start 110.617 115.443) (end 105.41 120.65) (width 0.8) (layer "F.Cu") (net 17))
 (segment (start 122.047 115.443) (end 110.617 115.443) (width 0.8) (layer "F.Cu") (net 17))
 (segment (start 105.41 120.65) (end 105.41 127.7525) (width 0.8) (layer "F.Cu") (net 17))
 (via (at 124.46 113.03) (size 1.8) (drill 0.9) (layers "F.Cu" "B.Cu") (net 17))
 (segment (start 124.46 102.87) (end 124.46 113.03) (width 0.8) (layer "B.Cu") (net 17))
 (segment (start 125.73 101.6) (end 124.46 102.87) (width 0.8) (layer "B.Cu") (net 17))
 (segment (start 127.3025 101.6) (end 125.73 101.6) (width 0.8) (layer "B.Cu") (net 17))
 (segment (start 111.76 118.11) (end 107.95 121.92) (width 0.8) (layer "F.Cu") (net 18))
 (segment (start 133.35 107.95) (end 133.35 93.98) (width 0.8) (layer "F.Cu") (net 18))
 (segment (start 107.95 121.92) (end 107.95 127.7525) (width 0.8) (layer "F.Cu") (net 18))
 (segment (start 113.03 118.11) (end 111.76 118.11) (width 0.8) (layer "F.Cu") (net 18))
 (via (at 133.35 107.95) (size 1.8) (drill 0.9) (layers "F.Cu" "B.Cu") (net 18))
 (via (at 113.03 118.11) (size 1.8) (drill 0.9) (layers "F.Cu" "B.Cu") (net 18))
 (via (at 133.35 93.98) (size 1.8) (drill 0.9) (layers "F.Cu" "B.Cu") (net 18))
 (segment (start 127.3025 93.98) (end 133.35 93.98) (width 0.8) (layer "B.Cu") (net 18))
 (segment (start 113.03 118.11) (end 123.19 118.11) (width 0.8) (layer "B.Cu") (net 18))
 (segment (start 123.19 118.11) (end 133.35 107.95) (width 0.8) (layer "B.Cu") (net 18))
 (segment (start 118.11 91.44) (end 119.6825 91.44) (width 0.8) (layer "F.Cu") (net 14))
 (segment (start 116.84 104.14) (end 116.84 92.71) (width 0.8) (layer "F.Cu") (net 14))
 (segment (start 116.84 92.71) (end 118.11 91.44) (width 0.8) (layer "F.Cu") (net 14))
 (via (at 116.84 104.14) (size 1.8) (drill 0.9) (layers "F.Cu" "B.Cu") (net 14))
 (segment (start 110.49 115.57) (end 110.49 127.7525) (width 0.8) (layer "B.Cu") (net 14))
 (segment (start 116.84 109.22) (end 110.49 115.57) (width 0.8) (layer "B.Cu") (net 14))
 (segment (start 116.84 104.14) (end 116.84 109.22) (width 0.8) (layer "B.Cu") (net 14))
 (segment (start 139.7 112.395) (end 131.445 112.395) (width 0.8) (layer "F.Cu") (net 20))
 (segment (start 113.03 123.19) (end 113.03 127.7525) (width 0.8) (layer "F.Cu") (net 20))
 (segment (start 116.84 119.38) (end 113.03 123.19) (width 0.8) (layer "F.Cu") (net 20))
 (segment (start 131.445 112.395) (end 124.46 119.38) (width 0.8) (layer "F.Cu") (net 20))
 (segment (start 124.46 119.38) (end 116.84 119.38) (width 0.8) (layer "F.Cu") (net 20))
 (via (at 139.7 112.395) (size 1.8) (drill 0.9) (layers "F.Cu" "B.Cu") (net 20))
 (segment (start 139.7 112.395) (end 139.7 102.87) (width 0.8) (layer "B.Cu") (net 20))
 (segment (start 139.7 102.87) (end 140.985 101.585) (width 0.8) (layer "B.Cu") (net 20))
 (segment (start 140.985 101.585) (end 142.225 101.585) (width 0.8) (layer "B.Cu") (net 20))
 (segment (start 144.353622 114.3) (end 132.08 114.3) (width 0.8) (layer "F.Cu") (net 22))
 (segment (start 125.73 120.65) (end 118.11 120.65) (width 0.8) (layer "F.Cu") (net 22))
 (segment (start 115.57 123.19) (end 115.57 127.7525) (width 0.8) (layer "F.Cu") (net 22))
 (segment (start 118.11 120.65) (end 115.57 123.19) (width 0.8) (layer "F.Cu") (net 22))
 (segment (start 149.845 101.585) (end 149.445 101.585) (width 0.8) (layer "F.Cu") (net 22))
 (segment (start 132.08 114.3) (end 125.73 120.65) (width 0.8) (layer "F.Cu") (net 22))
 (segment (start 147.32 111.333622) (end 144.353622 114.3) (width 0.8) (layer "F.Cu") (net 22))
 (segment (start 147.32 103.71) (end 147.32 111.333622) (width 0.8) (layer "F.Cu") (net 22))
 (segment (start 149.445 101.585) (end 147.32 103.71) (width 0.8) (layer "F.Cu") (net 22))
 (segment (start 118.11 123.19) (end 119.38 121.92) (width 0.8) (layer "F.Cu") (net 23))
 (segment (start 127 121.92) (end 132.715 116.205) (width 0.8) (layer "F.Cu") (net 23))
 (segment (start 153.67 110.49) (end 153.67 93.98) (width 0.8) (layer "F.Cu") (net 23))
 (segment (start 119.38 121.92) (end 127 121.92) (width 0.8) (layer "F.Cu") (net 23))
 (segment (start 118.11 127.7525) (end 118.11 123.19) (width 0.8) (layer "F.Cu") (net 23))
 (segment (start 147.955 116.205) (end 153.67 110.49) (width 0.8) (layer "F.Cu") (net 23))
 (segment (start 132.715 116.205) (end 147.955 116.205) (width 0.8) (layer "F.Cu") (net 23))
 (via (at 153.67 93.98) (size 1.8) (drill 0.9) (layers "F.Cu" "B.Cu") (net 23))
 (segment (start 153.67 93.98) (end 149.86 93.98) (width 0.8) (layer "B.Cu") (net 23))
 (segment (start 149.86 93.98) (end 149.845 93.965) (width 0.8) (layer "B.Cu") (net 23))
 (segment (start 144.78 109.22) (end 144.78 92.71) (width 0.8) (layer "F.Cu") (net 19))
 (segment (start 120.65 127.7525) (end 120.65 124.46) (width 0.8) (layer "F.Cu") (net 19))
 (segment (start 128.27 123.19) (end 133.35 118.11) (width 0.8) (layer "F.Cu") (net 19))
 (segment (start 142.24 111.76) (end 144.78 109.22) (width 0.8) (layer "F.Cu") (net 19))
 (segment (start 121.92 123.19) (end 128.27 123.19) (width 0.8) (layer "F.Cu") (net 19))
 (segment (start 120.65 124.46) (end 121.92 123.19) (width 0.8) (layer "F.Cu") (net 19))
 (segment (start 143.51 91.44) (end 142.24 91.44) (width 0.8) (layer "F.Cu") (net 19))
 (segment (start 144.78 92.71) (end 143.51 91.44) (width 0.8) (layer "F.Cu") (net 19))
 (segment (start 142.24 91.44) (end 142.225 91.425) (width 0.8) (layer "F.Cu") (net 19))
 (segment (start 133.35 118.11) (end 142.24 118.11) (width 0.8) (layer "F.Cu") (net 19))
 (via (at 142.24 111.76) (size 1.8) (drill 0.9) (layers "F.Cu" "B.Cu") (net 19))
 (via (at 142.24 118.11) (size 1.8) (drill 0.9) (layers "F.Cu" "B.Cu") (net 19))
 (segment (start 142.24 111.76) (end 142.24 118.11) (width 0.8) (layer "B.Cu") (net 19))
 (segment (start 97.14 101.6) (end 96.52 101.6) (width 0.8) (layer "F.Cu") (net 3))
 (segment (start 96.52 101.6) (end 92.71 105.41) (width 0.8) (layer "F.Cu") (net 3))
 (segment (start 92.71 105.41) (end 92.71 127.7525) (width 0.8) (layer "F.Cu") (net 3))
 (segment (start 95.25 119.38) (end 101.6 113.03) (width 0.8) (layer "B.Cu") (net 7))
 (segment (start 104.76 101.6) (end 102.87 101.6) (width 0.8) (layer "B.Cu") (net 7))
 (segment (start 102.87 101.6) (end 101.6 102.87) (width 0.8) (layer "B.Cu") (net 7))
 (segment (start 95.25 127.7525) (end 95.25 119.38) (width 0.8) (layer "B.Cu") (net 7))
 (segment (start 101.6 102.87) (end 101.6 113.03) (width 0.8) (layer "B.Cu") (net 7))
 (segment (start 109.22 93.98) (end 109.22 107.95) (width 0.8) (layer "F.Cu") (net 8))
 (via (at 109.22 93.98) (size 1.8) (drill 0.9) (layers "F.Cu" "B.Cu") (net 8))
 (via (at 109.22 107.95) (size 1.8) (drill 0.9) (layers "F.Cu" "B.Cu") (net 8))
 (segment (start 109.22 107.95) (end 97.79 119.38) (width 0.8) (layer "B.Cu") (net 8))
 (segment (start 104.76 93.98) (end 109.22 93.98) (width 0.8) (layer "B.Cu") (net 8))
 (segment (start 97.79 119.38) (end 97.79 127.7525) (width 0.8) (layer "B.Cu") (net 8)))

